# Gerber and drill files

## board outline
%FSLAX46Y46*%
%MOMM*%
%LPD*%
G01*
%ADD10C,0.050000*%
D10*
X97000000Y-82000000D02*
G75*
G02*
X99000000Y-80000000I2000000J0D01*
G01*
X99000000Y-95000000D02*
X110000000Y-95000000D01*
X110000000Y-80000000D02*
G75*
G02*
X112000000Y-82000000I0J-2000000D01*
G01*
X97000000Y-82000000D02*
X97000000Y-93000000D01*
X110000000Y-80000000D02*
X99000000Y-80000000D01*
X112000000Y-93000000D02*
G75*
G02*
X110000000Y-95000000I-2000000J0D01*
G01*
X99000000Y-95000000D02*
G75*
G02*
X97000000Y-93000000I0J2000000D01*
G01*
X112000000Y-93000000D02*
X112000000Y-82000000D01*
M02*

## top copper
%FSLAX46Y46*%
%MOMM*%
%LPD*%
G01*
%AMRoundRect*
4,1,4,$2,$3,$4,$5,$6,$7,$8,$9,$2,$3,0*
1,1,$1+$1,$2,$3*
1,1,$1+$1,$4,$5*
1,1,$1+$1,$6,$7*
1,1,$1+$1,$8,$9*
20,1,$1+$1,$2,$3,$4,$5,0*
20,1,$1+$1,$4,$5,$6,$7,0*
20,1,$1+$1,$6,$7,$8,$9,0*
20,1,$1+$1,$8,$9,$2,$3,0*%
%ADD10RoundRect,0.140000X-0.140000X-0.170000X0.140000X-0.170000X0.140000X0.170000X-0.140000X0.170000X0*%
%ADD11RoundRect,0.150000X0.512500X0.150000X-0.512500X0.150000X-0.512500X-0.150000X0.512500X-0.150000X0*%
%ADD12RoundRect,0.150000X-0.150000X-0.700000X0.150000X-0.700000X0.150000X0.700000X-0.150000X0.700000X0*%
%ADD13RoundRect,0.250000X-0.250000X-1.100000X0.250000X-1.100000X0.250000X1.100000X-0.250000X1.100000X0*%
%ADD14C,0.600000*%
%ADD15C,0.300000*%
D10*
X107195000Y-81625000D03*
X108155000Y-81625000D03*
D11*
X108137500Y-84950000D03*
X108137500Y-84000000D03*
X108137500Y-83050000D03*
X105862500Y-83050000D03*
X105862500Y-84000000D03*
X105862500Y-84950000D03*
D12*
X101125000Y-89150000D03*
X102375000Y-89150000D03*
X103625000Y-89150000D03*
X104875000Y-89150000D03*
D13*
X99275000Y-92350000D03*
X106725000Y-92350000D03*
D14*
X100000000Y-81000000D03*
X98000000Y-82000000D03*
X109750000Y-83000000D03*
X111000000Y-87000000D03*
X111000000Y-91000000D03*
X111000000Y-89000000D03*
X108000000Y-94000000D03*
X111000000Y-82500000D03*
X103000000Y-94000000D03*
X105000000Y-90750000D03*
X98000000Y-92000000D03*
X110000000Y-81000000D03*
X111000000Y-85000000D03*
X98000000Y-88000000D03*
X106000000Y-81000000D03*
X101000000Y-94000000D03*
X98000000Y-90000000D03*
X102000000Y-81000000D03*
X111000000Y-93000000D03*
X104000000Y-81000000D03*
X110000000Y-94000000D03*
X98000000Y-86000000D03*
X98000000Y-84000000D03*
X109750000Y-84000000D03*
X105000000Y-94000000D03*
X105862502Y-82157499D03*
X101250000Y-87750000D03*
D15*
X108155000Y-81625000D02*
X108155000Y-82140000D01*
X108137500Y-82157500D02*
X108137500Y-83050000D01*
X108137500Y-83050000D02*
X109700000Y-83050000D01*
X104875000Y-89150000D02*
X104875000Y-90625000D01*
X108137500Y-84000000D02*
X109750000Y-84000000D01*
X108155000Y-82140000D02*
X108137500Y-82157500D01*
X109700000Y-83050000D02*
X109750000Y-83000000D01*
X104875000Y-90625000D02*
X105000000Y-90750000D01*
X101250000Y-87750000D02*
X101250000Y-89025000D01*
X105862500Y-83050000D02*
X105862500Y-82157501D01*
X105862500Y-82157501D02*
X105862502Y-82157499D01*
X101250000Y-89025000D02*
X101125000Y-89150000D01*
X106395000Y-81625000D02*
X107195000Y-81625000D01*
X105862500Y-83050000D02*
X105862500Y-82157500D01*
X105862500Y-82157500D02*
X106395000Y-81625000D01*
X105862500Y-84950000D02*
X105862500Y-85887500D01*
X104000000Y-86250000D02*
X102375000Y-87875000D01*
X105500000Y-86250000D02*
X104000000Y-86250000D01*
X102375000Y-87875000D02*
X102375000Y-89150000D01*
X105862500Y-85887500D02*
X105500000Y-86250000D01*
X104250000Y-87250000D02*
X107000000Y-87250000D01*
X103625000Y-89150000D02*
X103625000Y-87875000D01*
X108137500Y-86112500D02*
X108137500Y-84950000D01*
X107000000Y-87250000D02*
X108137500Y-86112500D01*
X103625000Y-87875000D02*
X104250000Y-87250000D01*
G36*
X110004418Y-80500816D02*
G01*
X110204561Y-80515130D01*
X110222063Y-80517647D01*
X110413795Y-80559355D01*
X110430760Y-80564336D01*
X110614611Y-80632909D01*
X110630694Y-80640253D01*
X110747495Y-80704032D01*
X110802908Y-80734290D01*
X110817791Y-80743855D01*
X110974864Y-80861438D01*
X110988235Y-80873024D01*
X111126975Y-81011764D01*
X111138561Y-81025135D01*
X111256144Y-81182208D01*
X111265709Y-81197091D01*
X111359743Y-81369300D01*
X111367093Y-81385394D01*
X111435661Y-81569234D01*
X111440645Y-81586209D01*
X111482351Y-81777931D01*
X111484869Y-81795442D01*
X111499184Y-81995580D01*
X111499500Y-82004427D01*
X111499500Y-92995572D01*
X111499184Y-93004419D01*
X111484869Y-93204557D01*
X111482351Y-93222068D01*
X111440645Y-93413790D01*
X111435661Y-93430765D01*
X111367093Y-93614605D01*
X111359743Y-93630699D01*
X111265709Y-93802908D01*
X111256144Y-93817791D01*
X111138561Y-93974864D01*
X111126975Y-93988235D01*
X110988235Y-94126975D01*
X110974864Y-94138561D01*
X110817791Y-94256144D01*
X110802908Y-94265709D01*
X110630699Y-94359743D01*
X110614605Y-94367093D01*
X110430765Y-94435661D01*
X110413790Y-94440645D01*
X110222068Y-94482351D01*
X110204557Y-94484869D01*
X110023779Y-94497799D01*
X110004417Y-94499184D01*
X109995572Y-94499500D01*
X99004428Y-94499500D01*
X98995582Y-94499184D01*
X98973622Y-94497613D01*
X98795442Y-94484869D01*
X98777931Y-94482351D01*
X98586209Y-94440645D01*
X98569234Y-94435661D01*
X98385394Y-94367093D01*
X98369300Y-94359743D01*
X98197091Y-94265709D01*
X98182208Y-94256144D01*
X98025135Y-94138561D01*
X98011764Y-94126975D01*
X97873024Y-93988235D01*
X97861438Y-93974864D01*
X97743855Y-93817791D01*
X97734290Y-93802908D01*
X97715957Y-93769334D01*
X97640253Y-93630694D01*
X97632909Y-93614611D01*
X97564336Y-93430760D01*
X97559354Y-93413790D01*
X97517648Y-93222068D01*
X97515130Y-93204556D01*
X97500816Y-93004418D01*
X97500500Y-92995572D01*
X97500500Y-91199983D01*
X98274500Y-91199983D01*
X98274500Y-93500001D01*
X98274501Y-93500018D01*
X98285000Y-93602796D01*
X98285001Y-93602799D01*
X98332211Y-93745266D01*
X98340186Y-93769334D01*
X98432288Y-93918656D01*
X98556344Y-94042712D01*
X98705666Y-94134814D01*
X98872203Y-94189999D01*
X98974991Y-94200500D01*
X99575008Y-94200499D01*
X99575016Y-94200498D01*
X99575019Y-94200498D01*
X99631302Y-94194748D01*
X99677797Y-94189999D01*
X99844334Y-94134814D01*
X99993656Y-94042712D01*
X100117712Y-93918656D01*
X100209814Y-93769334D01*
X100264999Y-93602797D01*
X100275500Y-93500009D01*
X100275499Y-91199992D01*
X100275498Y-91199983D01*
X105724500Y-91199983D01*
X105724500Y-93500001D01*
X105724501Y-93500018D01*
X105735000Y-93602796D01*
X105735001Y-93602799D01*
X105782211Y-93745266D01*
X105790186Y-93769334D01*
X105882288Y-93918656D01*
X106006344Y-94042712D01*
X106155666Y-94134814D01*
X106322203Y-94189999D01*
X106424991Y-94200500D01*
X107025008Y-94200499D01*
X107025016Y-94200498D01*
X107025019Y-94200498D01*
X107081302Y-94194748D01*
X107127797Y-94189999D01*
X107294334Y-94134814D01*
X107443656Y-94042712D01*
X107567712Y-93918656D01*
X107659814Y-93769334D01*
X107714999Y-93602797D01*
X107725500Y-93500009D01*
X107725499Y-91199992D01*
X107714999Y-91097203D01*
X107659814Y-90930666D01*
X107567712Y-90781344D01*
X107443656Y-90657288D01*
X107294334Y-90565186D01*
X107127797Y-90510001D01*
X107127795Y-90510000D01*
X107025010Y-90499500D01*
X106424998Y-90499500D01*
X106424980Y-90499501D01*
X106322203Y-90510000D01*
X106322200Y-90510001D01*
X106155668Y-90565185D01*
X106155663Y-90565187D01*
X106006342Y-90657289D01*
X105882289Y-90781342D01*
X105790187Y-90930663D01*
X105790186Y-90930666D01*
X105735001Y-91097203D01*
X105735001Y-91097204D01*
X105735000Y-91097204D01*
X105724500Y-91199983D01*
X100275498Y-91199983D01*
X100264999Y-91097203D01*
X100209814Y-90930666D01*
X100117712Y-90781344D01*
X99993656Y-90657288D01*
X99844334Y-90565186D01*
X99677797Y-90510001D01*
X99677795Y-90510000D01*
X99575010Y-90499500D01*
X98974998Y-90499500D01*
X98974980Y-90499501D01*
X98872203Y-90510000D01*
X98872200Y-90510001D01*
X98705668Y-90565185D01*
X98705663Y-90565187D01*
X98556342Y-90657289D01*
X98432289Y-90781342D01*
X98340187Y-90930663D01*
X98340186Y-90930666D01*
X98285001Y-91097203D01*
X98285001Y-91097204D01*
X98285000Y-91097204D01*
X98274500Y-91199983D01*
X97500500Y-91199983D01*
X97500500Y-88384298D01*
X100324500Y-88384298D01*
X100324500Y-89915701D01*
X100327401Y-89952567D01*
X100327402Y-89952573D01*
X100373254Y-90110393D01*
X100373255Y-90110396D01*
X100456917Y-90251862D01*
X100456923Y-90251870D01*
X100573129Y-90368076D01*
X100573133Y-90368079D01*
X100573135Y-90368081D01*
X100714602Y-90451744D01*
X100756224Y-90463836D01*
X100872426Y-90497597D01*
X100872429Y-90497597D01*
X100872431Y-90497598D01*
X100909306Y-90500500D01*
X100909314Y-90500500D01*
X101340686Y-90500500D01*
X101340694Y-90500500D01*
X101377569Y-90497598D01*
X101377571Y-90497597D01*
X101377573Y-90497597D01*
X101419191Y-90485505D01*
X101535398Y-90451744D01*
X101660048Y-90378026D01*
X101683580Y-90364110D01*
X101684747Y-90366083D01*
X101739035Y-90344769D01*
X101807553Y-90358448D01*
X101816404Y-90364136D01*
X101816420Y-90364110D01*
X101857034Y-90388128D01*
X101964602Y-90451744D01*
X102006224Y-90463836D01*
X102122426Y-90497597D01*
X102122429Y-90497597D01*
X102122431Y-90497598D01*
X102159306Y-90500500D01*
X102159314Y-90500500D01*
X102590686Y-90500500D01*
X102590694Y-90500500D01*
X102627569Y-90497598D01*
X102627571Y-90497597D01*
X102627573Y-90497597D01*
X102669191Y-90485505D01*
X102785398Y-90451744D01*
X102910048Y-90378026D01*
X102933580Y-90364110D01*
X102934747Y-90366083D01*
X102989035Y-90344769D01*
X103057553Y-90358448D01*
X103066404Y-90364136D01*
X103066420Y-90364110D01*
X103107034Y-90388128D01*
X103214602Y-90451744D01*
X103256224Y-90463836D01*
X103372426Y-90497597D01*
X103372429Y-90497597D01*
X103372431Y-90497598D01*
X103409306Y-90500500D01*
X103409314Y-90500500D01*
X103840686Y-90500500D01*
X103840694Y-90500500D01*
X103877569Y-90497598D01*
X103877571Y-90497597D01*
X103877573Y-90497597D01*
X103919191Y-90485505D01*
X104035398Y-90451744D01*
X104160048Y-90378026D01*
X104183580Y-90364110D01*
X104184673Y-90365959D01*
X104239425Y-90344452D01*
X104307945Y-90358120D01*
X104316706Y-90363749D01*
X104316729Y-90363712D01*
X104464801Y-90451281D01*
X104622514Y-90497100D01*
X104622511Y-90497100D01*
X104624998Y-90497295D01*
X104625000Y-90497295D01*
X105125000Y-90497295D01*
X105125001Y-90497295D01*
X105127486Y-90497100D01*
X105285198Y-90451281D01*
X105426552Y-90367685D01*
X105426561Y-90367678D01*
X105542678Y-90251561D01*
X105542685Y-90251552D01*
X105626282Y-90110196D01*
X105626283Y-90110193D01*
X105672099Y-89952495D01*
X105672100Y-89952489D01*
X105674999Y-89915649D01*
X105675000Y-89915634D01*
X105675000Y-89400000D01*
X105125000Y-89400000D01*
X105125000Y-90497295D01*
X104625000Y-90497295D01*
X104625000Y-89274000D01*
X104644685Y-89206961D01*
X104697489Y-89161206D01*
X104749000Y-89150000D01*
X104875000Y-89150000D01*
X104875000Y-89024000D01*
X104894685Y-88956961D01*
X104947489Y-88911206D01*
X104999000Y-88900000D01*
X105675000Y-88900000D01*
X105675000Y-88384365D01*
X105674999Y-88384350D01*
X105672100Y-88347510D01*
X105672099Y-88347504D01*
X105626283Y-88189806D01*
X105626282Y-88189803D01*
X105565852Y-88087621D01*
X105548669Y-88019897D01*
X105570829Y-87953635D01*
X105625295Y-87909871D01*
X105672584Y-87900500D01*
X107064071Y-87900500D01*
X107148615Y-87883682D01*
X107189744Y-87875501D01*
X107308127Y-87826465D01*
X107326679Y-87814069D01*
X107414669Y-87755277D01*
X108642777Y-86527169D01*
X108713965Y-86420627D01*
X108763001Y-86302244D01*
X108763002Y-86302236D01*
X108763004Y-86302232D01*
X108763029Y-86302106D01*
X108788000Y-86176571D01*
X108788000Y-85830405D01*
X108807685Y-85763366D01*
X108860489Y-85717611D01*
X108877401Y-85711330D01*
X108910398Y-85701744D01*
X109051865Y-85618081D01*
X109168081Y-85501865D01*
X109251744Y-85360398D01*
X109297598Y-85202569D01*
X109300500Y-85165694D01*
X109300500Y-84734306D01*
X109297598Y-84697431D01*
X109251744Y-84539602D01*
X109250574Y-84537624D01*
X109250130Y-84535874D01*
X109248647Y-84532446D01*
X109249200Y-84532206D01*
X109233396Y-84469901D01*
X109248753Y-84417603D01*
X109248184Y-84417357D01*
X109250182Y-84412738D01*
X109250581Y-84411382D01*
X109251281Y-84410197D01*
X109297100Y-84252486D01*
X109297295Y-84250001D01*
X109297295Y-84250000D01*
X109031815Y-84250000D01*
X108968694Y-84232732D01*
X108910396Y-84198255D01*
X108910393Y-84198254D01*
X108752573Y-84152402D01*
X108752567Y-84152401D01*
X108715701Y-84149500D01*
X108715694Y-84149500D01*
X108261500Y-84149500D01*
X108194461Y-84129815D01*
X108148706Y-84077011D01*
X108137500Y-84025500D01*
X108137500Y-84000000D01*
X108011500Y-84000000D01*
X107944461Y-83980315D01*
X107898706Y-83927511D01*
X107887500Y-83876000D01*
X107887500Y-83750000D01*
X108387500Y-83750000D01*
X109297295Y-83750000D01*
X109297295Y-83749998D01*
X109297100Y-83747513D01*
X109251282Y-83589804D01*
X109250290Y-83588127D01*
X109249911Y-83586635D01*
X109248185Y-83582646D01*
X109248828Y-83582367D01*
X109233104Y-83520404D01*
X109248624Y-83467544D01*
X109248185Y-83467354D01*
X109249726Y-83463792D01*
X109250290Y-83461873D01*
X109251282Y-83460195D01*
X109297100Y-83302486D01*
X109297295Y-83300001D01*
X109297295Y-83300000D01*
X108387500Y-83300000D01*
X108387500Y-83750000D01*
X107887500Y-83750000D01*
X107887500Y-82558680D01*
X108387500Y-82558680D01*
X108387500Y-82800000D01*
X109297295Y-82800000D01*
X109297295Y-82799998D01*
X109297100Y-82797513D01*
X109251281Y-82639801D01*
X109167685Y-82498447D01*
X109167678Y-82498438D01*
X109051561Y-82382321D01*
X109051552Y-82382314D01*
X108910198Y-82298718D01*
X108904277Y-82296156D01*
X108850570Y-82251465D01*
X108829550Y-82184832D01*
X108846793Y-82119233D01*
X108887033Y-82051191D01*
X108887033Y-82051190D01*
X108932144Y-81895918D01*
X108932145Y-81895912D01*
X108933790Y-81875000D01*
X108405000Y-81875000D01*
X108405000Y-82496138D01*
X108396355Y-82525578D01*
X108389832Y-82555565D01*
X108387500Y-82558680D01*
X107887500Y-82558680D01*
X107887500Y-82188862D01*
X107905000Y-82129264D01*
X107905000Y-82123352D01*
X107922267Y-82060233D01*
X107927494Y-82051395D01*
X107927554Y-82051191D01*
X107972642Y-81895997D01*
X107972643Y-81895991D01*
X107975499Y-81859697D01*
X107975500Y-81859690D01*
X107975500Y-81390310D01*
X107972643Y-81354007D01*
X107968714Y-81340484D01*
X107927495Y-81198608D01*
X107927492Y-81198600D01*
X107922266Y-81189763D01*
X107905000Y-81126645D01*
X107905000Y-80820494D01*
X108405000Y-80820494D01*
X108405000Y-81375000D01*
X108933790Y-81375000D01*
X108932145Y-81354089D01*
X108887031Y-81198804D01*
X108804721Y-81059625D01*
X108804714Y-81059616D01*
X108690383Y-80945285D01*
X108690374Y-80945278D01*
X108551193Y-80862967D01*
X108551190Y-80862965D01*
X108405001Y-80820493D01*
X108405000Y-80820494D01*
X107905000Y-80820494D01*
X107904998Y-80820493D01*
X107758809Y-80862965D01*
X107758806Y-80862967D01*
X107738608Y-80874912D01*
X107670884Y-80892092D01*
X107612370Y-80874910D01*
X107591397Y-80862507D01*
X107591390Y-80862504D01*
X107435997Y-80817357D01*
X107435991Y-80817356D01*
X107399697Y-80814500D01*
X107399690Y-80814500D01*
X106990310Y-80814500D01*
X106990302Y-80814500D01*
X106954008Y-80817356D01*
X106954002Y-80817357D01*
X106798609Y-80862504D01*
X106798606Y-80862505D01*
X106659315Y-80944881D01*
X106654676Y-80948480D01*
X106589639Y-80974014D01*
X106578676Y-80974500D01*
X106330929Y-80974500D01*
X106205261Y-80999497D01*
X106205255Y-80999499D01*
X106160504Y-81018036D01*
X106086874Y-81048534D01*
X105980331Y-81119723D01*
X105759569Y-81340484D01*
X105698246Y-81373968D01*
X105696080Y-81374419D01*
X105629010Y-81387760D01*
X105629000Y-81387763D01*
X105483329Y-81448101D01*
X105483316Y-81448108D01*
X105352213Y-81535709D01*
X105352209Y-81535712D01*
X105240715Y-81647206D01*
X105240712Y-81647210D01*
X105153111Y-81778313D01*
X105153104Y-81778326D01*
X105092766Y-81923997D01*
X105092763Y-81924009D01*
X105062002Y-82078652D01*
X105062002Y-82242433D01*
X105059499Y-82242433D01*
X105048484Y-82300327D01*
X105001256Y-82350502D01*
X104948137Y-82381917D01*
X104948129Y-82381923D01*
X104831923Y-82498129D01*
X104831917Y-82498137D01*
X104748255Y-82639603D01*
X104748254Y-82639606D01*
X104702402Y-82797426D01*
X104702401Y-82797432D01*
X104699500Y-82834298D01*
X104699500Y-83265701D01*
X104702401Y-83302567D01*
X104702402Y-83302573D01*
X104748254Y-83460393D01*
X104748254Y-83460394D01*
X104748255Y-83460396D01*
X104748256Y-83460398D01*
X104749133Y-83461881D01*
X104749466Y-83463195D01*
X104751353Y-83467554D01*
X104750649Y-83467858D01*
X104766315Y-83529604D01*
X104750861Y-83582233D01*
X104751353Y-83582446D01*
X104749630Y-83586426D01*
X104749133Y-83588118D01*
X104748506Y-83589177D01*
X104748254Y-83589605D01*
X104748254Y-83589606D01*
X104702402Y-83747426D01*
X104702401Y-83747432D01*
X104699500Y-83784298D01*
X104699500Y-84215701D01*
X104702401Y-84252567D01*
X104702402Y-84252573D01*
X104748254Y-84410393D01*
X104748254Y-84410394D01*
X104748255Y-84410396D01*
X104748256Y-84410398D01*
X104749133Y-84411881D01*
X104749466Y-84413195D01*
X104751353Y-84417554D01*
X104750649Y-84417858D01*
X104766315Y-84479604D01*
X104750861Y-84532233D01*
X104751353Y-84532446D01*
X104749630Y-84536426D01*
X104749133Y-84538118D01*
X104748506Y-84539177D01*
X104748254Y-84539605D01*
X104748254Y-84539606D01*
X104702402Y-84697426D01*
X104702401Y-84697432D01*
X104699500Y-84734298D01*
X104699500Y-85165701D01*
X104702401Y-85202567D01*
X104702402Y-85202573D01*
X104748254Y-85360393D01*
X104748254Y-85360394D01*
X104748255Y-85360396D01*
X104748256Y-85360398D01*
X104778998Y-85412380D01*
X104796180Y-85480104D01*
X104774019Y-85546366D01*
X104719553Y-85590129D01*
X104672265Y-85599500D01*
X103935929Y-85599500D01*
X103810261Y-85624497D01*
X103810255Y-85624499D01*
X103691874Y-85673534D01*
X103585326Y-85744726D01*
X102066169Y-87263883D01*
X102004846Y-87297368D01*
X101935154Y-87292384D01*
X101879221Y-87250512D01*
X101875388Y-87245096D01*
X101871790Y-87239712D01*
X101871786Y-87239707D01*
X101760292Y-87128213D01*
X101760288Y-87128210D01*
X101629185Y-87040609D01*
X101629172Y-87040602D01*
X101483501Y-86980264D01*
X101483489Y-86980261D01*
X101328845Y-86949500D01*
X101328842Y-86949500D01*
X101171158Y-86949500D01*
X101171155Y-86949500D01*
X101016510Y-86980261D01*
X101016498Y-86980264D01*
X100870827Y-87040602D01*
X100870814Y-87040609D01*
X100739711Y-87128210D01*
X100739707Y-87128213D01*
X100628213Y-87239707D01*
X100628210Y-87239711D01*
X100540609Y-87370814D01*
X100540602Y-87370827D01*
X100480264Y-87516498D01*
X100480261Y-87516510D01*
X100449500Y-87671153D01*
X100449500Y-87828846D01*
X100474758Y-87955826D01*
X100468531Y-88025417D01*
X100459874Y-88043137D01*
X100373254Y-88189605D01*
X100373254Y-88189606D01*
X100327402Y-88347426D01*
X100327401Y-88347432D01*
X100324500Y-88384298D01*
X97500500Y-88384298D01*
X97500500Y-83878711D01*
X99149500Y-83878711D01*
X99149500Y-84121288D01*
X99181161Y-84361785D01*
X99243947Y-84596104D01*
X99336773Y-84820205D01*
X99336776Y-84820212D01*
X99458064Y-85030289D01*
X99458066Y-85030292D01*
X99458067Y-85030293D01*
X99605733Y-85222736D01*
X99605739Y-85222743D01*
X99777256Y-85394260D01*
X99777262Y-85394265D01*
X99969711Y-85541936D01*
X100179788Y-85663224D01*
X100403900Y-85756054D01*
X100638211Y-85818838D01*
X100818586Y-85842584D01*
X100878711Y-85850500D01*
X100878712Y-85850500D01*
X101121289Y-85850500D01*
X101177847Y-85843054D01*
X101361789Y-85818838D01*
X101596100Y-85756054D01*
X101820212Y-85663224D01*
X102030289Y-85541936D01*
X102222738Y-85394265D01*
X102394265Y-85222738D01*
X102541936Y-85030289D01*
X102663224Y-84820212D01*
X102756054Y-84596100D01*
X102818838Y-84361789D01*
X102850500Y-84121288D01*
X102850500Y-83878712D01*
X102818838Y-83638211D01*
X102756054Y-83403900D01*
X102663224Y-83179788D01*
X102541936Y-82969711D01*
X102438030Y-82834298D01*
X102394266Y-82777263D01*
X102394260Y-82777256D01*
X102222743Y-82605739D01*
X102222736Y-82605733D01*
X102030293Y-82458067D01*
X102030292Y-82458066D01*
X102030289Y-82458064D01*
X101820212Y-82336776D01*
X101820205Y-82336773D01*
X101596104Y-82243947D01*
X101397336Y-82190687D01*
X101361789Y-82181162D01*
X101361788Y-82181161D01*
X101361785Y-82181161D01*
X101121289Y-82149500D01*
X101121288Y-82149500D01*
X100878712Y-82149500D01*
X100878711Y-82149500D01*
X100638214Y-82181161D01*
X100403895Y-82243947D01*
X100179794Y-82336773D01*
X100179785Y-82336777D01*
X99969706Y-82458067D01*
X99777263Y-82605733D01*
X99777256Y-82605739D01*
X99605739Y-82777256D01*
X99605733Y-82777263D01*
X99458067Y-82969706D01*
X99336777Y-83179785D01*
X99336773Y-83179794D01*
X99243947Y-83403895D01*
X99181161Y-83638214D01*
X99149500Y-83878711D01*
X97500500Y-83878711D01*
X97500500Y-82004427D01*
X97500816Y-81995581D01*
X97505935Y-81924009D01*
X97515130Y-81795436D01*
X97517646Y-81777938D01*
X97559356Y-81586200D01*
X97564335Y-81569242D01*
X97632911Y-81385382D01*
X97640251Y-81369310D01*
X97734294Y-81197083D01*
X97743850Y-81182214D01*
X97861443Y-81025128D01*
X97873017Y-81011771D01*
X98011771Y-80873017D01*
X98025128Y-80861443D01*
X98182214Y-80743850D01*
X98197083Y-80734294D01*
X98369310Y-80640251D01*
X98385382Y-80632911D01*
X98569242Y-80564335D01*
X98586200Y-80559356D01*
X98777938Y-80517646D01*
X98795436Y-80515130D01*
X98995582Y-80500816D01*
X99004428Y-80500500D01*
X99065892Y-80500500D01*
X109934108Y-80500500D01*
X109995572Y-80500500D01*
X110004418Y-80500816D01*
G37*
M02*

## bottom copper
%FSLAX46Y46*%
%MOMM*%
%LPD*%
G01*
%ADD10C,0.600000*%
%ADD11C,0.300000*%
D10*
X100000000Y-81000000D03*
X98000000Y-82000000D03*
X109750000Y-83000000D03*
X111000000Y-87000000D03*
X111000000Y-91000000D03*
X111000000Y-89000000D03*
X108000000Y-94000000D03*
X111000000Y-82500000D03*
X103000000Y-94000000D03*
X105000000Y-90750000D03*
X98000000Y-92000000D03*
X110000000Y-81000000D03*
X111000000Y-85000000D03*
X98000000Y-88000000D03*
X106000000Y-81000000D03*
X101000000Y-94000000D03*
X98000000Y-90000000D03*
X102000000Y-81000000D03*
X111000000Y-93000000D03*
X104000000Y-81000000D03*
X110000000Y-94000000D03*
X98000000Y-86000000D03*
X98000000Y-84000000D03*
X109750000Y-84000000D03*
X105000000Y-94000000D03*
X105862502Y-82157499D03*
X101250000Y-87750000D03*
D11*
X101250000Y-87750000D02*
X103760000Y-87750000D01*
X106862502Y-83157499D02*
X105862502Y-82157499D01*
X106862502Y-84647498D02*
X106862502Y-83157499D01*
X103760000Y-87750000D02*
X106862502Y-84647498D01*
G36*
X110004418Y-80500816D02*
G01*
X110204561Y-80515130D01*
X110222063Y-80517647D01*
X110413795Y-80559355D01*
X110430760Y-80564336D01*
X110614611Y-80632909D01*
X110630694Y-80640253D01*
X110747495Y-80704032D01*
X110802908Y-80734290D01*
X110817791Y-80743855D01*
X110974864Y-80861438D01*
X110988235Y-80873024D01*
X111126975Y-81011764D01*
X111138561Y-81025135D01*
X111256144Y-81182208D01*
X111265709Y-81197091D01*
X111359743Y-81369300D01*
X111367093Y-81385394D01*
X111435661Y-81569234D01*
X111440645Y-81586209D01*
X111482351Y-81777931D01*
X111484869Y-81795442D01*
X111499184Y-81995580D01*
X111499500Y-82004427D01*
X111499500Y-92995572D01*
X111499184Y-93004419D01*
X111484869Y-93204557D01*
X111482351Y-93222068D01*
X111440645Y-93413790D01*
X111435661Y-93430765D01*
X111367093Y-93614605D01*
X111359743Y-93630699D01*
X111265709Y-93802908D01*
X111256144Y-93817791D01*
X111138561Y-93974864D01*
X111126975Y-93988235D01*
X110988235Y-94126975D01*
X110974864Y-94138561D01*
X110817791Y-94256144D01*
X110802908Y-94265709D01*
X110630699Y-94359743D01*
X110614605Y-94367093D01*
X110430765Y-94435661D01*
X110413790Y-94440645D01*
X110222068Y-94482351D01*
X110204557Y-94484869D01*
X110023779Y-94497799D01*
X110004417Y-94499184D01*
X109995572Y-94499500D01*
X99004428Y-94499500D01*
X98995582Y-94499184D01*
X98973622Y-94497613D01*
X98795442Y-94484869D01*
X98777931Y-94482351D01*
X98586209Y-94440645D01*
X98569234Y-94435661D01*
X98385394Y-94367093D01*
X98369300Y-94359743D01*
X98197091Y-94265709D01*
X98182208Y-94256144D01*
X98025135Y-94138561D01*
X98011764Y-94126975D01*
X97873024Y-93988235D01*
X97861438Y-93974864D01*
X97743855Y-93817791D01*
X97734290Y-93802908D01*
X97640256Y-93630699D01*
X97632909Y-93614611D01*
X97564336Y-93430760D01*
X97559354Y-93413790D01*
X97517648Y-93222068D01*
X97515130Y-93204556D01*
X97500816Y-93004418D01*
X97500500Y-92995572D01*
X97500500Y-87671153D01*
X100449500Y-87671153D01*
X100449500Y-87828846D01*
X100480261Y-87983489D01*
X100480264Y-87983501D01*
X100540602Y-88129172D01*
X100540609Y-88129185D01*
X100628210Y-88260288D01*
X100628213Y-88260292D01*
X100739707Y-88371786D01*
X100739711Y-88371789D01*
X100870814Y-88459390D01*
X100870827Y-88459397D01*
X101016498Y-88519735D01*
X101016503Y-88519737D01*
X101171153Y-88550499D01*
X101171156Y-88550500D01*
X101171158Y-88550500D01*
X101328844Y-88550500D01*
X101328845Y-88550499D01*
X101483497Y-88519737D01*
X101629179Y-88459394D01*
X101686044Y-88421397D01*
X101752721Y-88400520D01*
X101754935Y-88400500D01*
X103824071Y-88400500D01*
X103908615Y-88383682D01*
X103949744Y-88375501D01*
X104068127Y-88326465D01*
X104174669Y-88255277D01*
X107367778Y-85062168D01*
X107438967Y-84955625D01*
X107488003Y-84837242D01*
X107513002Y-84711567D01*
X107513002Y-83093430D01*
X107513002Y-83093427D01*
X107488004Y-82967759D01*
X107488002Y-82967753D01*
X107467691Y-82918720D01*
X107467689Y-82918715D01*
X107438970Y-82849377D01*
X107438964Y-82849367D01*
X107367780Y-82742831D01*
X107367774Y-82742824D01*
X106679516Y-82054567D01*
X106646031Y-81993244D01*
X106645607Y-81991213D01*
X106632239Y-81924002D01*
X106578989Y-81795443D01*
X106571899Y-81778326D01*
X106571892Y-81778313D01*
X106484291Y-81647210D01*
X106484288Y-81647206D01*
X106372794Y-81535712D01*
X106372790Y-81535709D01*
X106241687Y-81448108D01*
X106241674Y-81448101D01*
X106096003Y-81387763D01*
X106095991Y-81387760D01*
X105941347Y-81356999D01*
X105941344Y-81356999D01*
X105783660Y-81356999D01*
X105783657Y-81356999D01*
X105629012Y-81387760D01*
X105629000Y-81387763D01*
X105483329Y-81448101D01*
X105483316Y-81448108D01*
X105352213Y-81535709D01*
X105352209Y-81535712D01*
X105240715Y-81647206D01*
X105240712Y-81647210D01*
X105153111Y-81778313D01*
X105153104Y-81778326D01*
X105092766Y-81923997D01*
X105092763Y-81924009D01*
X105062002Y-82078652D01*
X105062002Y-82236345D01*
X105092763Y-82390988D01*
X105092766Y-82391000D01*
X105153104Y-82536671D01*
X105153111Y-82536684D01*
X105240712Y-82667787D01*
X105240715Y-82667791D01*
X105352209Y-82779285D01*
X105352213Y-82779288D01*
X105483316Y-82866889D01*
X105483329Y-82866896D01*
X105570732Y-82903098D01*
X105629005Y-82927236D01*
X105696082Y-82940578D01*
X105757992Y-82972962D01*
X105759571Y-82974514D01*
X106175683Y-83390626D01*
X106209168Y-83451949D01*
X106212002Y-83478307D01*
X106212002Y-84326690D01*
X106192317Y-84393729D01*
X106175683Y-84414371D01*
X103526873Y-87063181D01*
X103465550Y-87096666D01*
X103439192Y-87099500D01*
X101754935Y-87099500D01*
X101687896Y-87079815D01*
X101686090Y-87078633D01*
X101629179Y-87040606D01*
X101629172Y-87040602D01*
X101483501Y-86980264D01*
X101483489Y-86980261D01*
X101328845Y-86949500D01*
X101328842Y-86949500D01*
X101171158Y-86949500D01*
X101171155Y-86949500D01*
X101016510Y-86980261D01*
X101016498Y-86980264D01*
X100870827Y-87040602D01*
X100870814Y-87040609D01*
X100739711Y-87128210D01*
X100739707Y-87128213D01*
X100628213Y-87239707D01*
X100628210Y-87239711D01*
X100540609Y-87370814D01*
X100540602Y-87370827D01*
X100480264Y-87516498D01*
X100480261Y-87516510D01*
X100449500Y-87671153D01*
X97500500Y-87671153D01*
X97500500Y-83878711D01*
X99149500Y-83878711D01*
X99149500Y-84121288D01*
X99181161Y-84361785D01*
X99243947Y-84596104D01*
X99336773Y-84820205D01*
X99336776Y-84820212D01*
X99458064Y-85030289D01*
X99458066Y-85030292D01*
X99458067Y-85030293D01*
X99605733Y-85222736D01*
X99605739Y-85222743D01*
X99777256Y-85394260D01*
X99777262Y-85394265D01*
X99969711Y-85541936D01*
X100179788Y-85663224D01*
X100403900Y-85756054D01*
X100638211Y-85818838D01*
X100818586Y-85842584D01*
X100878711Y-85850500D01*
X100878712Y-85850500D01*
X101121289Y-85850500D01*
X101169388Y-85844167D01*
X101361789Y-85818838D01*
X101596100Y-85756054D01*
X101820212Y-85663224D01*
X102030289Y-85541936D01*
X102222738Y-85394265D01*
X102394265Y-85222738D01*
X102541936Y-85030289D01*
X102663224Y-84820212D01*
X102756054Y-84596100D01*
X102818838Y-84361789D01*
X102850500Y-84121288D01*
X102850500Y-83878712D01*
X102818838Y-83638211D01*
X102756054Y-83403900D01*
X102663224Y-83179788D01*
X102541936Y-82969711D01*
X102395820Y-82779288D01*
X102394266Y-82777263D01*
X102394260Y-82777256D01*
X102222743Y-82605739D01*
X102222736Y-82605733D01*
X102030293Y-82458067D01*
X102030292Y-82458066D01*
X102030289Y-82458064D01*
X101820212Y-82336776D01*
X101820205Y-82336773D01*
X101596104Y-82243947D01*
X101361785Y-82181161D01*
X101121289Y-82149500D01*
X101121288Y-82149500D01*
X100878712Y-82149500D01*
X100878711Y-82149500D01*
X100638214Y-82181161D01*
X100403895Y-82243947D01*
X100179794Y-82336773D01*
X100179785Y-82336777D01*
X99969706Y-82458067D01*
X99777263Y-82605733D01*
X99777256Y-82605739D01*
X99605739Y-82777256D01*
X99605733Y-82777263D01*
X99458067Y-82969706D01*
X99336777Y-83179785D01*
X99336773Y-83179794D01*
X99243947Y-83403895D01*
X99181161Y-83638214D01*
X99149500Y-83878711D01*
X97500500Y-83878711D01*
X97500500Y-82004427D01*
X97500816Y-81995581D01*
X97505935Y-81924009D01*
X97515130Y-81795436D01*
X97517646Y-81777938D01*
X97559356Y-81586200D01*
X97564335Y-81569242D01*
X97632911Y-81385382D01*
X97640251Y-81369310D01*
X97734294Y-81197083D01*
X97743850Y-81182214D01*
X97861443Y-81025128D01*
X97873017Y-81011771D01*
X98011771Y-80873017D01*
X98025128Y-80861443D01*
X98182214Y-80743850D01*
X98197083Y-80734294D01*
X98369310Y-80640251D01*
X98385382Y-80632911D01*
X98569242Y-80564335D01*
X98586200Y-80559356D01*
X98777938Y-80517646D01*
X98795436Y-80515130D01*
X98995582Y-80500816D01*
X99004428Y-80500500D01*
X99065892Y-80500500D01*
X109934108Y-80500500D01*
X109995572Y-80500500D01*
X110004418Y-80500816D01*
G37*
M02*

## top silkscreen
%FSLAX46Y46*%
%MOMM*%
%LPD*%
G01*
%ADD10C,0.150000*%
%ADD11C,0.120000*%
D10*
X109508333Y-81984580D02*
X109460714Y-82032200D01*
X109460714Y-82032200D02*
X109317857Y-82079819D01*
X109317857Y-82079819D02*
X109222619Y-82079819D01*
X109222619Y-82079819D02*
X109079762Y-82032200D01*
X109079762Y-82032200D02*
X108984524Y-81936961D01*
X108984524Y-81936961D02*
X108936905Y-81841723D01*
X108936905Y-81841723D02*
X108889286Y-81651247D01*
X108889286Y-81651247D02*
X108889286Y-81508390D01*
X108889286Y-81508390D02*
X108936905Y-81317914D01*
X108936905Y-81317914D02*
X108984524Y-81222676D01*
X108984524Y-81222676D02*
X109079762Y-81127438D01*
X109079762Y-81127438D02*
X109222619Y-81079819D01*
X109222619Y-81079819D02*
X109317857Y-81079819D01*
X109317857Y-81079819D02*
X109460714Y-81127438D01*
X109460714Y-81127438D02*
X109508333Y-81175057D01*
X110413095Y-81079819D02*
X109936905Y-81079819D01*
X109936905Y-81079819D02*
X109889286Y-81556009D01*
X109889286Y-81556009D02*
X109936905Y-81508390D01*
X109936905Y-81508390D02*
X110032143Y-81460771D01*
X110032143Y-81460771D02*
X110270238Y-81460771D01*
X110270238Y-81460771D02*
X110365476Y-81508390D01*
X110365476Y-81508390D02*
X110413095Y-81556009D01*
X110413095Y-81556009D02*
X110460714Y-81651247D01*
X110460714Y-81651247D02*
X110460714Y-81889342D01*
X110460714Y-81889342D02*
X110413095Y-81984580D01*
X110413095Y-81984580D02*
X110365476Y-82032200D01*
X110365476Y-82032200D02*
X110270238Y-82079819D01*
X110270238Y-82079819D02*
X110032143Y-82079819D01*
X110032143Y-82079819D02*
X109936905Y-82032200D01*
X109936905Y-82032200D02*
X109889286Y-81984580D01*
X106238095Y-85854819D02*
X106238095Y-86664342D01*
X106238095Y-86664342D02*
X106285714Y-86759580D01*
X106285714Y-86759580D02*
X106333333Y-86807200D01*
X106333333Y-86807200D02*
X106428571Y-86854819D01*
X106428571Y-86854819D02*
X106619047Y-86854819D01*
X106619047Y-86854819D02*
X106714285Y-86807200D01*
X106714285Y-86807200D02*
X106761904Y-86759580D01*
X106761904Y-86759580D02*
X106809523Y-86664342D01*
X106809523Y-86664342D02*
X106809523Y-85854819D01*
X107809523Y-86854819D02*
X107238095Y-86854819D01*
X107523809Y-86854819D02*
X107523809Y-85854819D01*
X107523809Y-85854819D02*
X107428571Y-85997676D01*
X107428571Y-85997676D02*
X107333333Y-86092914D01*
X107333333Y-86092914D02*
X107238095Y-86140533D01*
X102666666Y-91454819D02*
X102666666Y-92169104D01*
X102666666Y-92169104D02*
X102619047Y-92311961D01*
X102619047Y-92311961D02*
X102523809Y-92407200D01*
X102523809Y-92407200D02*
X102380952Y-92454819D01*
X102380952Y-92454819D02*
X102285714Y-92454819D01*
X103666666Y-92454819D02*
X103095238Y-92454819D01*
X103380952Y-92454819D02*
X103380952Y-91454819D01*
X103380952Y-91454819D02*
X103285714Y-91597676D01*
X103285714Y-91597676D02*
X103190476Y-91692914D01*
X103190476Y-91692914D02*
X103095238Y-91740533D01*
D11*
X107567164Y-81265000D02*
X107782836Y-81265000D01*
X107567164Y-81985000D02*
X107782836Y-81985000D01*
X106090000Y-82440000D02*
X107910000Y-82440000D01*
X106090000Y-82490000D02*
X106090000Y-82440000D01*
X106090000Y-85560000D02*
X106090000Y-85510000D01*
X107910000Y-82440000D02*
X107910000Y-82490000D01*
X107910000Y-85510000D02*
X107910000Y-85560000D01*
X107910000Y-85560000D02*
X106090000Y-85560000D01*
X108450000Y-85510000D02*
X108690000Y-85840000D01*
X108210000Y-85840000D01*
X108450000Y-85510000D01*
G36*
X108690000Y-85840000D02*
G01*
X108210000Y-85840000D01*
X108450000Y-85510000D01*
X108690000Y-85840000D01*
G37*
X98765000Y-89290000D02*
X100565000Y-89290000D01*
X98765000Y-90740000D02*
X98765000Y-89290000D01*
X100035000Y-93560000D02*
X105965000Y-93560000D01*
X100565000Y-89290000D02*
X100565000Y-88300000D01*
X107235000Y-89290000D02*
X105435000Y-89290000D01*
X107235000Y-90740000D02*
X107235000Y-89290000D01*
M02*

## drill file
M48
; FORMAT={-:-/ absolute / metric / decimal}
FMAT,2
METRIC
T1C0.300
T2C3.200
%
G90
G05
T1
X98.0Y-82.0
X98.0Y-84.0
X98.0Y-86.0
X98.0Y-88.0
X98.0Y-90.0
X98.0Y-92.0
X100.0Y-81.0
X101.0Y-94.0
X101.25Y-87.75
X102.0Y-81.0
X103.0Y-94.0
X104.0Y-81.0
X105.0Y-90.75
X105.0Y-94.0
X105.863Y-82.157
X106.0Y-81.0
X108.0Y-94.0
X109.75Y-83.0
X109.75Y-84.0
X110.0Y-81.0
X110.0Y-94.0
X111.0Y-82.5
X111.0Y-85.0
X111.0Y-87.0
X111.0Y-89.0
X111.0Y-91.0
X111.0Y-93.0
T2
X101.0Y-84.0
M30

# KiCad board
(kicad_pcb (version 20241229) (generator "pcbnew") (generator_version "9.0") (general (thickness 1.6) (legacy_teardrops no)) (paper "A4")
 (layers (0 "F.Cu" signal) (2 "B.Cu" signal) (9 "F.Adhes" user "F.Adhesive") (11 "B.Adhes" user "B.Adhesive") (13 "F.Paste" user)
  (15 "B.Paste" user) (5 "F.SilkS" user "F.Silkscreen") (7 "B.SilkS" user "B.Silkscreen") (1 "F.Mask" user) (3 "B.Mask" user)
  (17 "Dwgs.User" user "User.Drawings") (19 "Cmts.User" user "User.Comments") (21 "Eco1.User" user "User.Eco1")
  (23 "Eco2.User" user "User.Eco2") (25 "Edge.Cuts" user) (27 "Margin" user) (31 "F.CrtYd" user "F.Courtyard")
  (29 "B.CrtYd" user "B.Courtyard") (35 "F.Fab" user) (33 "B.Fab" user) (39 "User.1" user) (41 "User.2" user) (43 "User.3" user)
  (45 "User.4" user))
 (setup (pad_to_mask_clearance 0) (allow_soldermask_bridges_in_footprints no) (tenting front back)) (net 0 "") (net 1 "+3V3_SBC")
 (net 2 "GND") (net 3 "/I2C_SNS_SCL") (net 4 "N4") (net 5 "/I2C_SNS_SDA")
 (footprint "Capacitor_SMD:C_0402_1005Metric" (layer "F.Cu") (at 107.675 81.625)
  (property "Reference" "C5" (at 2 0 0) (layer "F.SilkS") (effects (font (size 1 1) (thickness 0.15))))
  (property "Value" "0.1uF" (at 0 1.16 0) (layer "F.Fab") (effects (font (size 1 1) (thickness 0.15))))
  (fp_line (start -0.107836 -0.36) (end 0.107836 -0.36) (stroke (width 0.12) (type solid)) (layer "F.SilkS"))
  (fp_line (start -0.107836 0.36) (end 0.107836 0.36) (stroke (width 0.12) (type solid)) (layer "F.SilkS"))
  (pad "1" smd roundrect (at -0.48 0) (size 0.56 0.62) (layers "F.Cu" "F.Mask" "F.Paste") (roundrect_rratio 0.25) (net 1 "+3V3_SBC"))
  (pad "2" smd roundrect (at 0.48 0) (size 0.56 0.62) (layers "F.Cu" "F.Mask" "F.Paste") (roundrect_rratio 0.25) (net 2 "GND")))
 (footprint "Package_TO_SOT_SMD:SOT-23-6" (layer "F.Cu") (at 107 84 180)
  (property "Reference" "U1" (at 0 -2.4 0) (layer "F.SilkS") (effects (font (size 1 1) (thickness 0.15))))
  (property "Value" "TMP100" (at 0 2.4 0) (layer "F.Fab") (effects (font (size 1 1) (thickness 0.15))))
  (fp_line (start 0.91 1.56) (end -0.91 1.56) (stroke (width 0.12) (type solid)) (layer "F.SilkS"))
  (fp_line (start 0.91 1.51) (end 0.91 1.56) (stroke (width 0.12) (type solid)) (layer "F.SilkS"))
  (fp_line (start 0.91 -1.56) (end 0.91 -1.51) (stroke (width 0.12) (type solid)) (layer "F.SilkS"))
  (fp_line (start -0.91 1.56) (end -0.91 1.51) (stroke (width 0.12) (type solid)) (layer "F.SilkS"))
  (fp_line (start -0.91 -1.51) (end -0.91 -1.56) (stroke (width 0.12) (type solid)) (layer "F.SilkS"))
  (fp_line (start -0.91 -1.56) (end 0.91 -1.56) (stroke (width 0.12) (type solid)) (layer "F.SilkS"))
  (fp_poly (pts (xy -1.45 -1.51) (xy -1.69 -1.84) (xy -1.21 -1.84)) (stroke (width 0.12) (type solid)) (fill yes) (layer "F.SilkS"))
  (pad "1" smd roundrect (at -1.1375 -0.95 180) (size 1.325 0.6) (layers "F.Cu" "F.Mask" "F.Paste") (roundrect_rratio 0.25)
   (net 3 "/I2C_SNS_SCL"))
  (pad "2" smd roundrect (at -1.1375 0 180) (size 1.325 0.6) (layers "F.Cu" "F.Mask" "F.Paste") (roundrect_rratio 0.25) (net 2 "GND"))
  (pad "3" smd roundrect (at -1.1375 0.95 180) (size 1.325 0.6) (layers "F.Cu" "F.Mask" "F.Paste") (roundrect_rratio 0.25) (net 2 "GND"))
  (pad "4" smd roundrect (at 1.1375 0.95 180) (size 1.325 0.6) (layers "F.Cu" "F.Mask" "F.Paste") (roundrect_rratio 0.25) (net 1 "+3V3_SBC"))
  (pad "5" smd roundrect (at 1.1375 0 180) (size 1.325 0.6) (layers "F.Cu" "F.Mask" "F.Paste") (roundrect_rratio 0.25) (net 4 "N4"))
  (pad "6" smd roundrect (at 1.1375 -0.95 180) (size 1.325 0.6) (layers "F.Cu" "F.Mask" "F.Paste") (roundrect_rratio 0.25)
   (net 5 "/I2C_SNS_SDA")))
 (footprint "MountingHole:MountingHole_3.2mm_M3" (layer "F.Cu") (at 101 84)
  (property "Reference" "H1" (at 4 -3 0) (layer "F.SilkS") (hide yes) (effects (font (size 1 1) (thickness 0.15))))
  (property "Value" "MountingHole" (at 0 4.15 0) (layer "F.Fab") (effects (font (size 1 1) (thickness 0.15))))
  (pad "" np_thru_hole circle (at 0 0) (size 3.2 3.2) (drill 3.2) (layers "*.Cu" "*.Mask")))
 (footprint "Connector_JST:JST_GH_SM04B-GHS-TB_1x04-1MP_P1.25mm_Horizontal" (layer "F.Cu") (at 103 91)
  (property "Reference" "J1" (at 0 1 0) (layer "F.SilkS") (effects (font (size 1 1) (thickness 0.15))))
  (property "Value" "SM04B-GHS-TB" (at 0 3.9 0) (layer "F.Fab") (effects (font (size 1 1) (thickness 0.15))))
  (fp_line (start -4.235 -1.71) (end -2.435 -1.71) (stroke (width 0.12) (type solid)) (layer "F.SilkS"))
  (fp_line (start -4.235 -0.26) (end -4.235 -1.71) (stroke (width 0.12) (type solid)) (layer "F.SilkS"))
  (fp_line (start -2.965 2.56) (end 2.965 2.56) (stroke (width 0.12) (type solid)) (layer "F.SilkS"))
  (fp_line (start -2.435 -1.71) (end -2.435 -2.7) (stroke (width 0.12) (type solid)) (layer "F.SilkS"))
  (fp_line (start 4.235 -1.71) (end 2.435 -1.71) (stroke (width 0.12) (type solid)) (layer "F.SilkS"))
  (fp_line (start 4.235 -0.26) (end 4.235 -1.71) (stroke (width 0.12) (type solid)) (layer "F.SilkS"))
  (pad "1" smd roundrect (at -1.875 -1.85) (size 0.6 1.7) (layers "F.Cu" "F.Mask" "F.Paste") (roundrect_rratio 0.25) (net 1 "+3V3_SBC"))
  (pad "2" smd roundrect (at -0.625 -1.85) (size 0.6 1.7) (layers "F.Cu" "F.Mask" "F.Paste") (roundrect_rratio 0.25) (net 5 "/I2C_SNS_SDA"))
  (pad "3" smd roundrect (at 0.625 -1.85) (size 0.6 1.7) (layers "F.Cu" "F.Mask" "F.Paste") (roundrect_rratio 0.25) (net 3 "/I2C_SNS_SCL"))
  (pad "4" smd roundrect (at 1.875 -1.85) (size 0.6 1.7) (layers "F.Cu" "F.Mask" "F.Paste") (roundrect_rratio 0.25) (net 2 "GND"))
  (pad "MP" smd roundrect (at -3.725 1.35) (size 1 2.7) (layers "F.Cu" "F.Mask" "F.Paste") (roundrect_rratio 0.25))
  (pad "MP" smd roundrect (at 3.725 1.35) (size 1 2.7) (layers "F.Cu" "F.Mask" "F.Paste") (roundrect_rratio 0.25)))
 (gr_arc (start 97 82) (mid 97.585786 80.585786) (end 99 80) (stroke (width 0.05) (type default)) (layer "Edge.Cuts"))
 (gr_line (start 99 95) (end 110 95) (stroke (width 0.05) (type default)) (layer "Edge.Cuts"))
 (gr_arc (start 110 80) (mid 111.414214 80.585786) (end 112 82) (stroke (width 0.05) (type default)) (layer "Edge.Cuts"))
 (gr_line (start 97 82) (end 97 93) (stroke (width 0.05) (type default)) (layer "Edge.Cuts"))
 (gr_line (start 110 80) (end 99 80) (stroke (width 0.05) (type default)) (layer "Edge.Cuts"))
 (gr_arc (start 112 93) (mid 111.414214 94.414214) (end 110 95) (stroke (width 0.05) (type default)) (layer "Edge.Cuts"))
 (gr_arc (start 99 95) (mid 97.585786 94.414214) (end 97 93) (stroke (width 0.05) (type default)) (layer "Edge.Cuts"))
 (gr_line (start 112 93) (end 112 82) (stroke (width 0.05) (type default)) (layer "Edge.Cuts"))
 (segment (start 108.155 81.625) (end 108.155 82.14) (width 0.3) (layer "F.Cu") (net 2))
 (segment (start 108.1375 82.1575) (end 108.1375 83.05) (width 0.3) (layer "F.Cu") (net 2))
 (segment (start 108.1375 83.05) (end 109.7 83.05) (width 0.3) (layer "F.Cu") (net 2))
 (segment (start 104.875 89.15) (end 104.875 90.625) (width 0.3) (layer "F.Cu") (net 2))
 (segment (start 108.1375 84) (end 109.75 84) (width 0.3) (layer "F.Cu") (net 2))
 (segment (start 108.155 82.14) (end 108.1375 82.1575) (width 0.3) (layer "F.Cu") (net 2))
 (segment (start 109.7 83.05) (end 109.75 83) (width 0.3) (layer "F.Cu") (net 2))
 (segment (start 104.875 90.625) (end 105 90.75) (width 0.3) (layer "F.Cu") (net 2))
 (via (at 100 81) (size 0.6) (drill 0.3) (layers "F.Cu" "B.Cu") (free yes) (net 2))
 (via (at 98 82) (size 0.6) (drill 0.3) (layers "F.Cu" "B.Cu") (free yes) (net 2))
 (via (at 109.75 83) (size 0.6) (drill 0.3) (layers "F.Cu" "B.Cu") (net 2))
 (via (at 111 87) (size 0.6) (drill 0.3) (layers "F.Cu" "B.Cu") (free yes) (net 2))
 (via (at 111 91) (size 0.6) (drill 0.3) (layers "F.Cu" "B.Cu") (free yes) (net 2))
 (via (at 111 89) (size 0.6) (drill 0.3) (layers "F.Cu" "B.Cu") (free yes) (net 2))
 (via (at 108 94) (size 0.6) (drill 0.3) (layers "F.Cu" "B.Cu") (free yes) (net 2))
 (via (at 111 82.5) (size 0.6) (drill 0.3) (layers "F.Cu" "B.Cu") (free yes) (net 2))
 (via (at 103 94) (size 0.6) (drill 0.3) (layers "F.Cu" "B.Cu") (free yes) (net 2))
 (via (at 105 90.75) (size 0.6) (drill 0.3) (layers "F.Cu" "B.Cu") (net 2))
 (via (at 98 92) (size 0.6) (drill 0.3) (layers "F.Cu" "B.Cu") (free yes) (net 2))
 (via (at 110 81) (size 0.6) (drill 0.3) (layers "F.Cu" "B.Cu") (free yes) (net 2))
 (via (at 111 85) (size 0.6) (drill 0.3) (layers "F.Cu" "B.Cu") (free yes) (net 2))
 (via (at 98 88) (size 0.6) (drill 0.3) (layers "F.Cu" "B.Cu") (free yes) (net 2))
 (via (at 106 81) (size 0.6) (drill 0.3) (layers "F.Cu" "B.Cu") (free yes) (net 2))
 (via (at 101 94) (size 0.6) (drill 0.3) (layers "F.Cu" "B.Cu") (free yes) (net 2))
 (via (at 98 90) (size 0.6) (drill 0.3) (layers "F.Cu" "B.Cu") (free yes) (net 2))
 (via (at 102 81) (size 0.6) (drill 0.3) (layers "F.Cu" "B.Cu") (free yes) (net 2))
 (via (at 111 93) (size 0.6) (drill 0.3) (layers "F.Cu" "B.Cu") (free yes) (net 2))
 (via (at 104 81) (size 0.6) (drill 0.3) (layers "F.Cu" "B.Cu") (free yes) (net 2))
 (via (at 110 94) (size 0.6) (drill 0.3) (layers "F.Cu" "B.Cu") (free yes) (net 2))
 (via (at 98 86) (size 0.6) (drill 0.3) (layers "F.Cu" "B.Cu") (free yes) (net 2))
 (via (at 98 84) (size 0.6) (drill 0.3) (layers "F.Cu" "B.Cu") (free yes) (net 2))
 (via (at 109.75 84) (size 0.6) (drill 0.3) (layers "F.Cu" "B.Cu") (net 2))
 (via (at 105 94) (size 0.6) (drill 0.3) (layers "F.Cu" "B.Cu") (free yes) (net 2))
 (segment (start 101.25 87.75) (end 101.25 89.025) (width 0.3) (layer "F.Cu") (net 1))
 (segment (start 105.8625 83.05) (end 105.8625 82.157501) (width 0.3) (layer "F.Cu") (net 1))
 (segment (start 105.8625 82.157501) (end 105.862502 82.157499) (width 0.3) (layer "F.Cu") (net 1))
 (segment (start 101.25 89.025) (end 101.125 89.15) (width 0.3) (layer "F.Cu") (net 1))
 (segment (start 106.395 81.625) (end 107.195 81.625) (width 0.3) (layer "F.Cu") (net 1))
 (segment (start 105.8625 83.05) (end 105.8625 82.1575) (width 0.3) (layer "F.Cu") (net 1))
 (segment (start 105.8625 82.1575) (end 106.395 81.625) (width 0.3) (layer "F.Cu") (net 1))
 (via (at 105.862502 82.157499) (size 0.6) (drill 0.3) (layers "F.Cu" "B.Cu") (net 1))
 (via (at 101.25 87.75) (size 0.6) (drill 0.3) (layers "F.Cu" "B.Cu") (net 1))
 (segment (start 101.25 87.75) (end 103.76 87.75) (width 0.3) (layer "B.Cu") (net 1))
 (segment (start 106.862502 83.157499) (end 105.862502 82.157499) (width 0.3) (layer "B.Cu") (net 1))
 (segment (start 106.862502 84.647498) (end 106.862502 83.157499) (width 0.3) (layer "B.Cu") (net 1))
 (segment (start 103.76 87.75) (end 106.862502 84.647498) (width 0.3) (layer "B.Cu") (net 1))
 (segment (start 105.8625 84.95) (end 105.8625 85.8875) (width 0.3) (layer "F.Cu") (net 5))
 (segment (start 104 86.25) (end 102.375 87.875) (width 0.3) (layer "F.Cu") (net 5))
 (segment (start 105.5 86.25) (end 104 86.25) (width 0.3) (layer "F.Cu") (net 5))
 (segment (start 102.375 87.875) (end 102.375 89.15) (width 0.3) (layer "F.Cu") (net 5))
 (segment (start 105.8625 85.8875) (end 105.5 86.25) (width 0.3) (layer "F.Cu") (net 5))
 (segment (start 104.25 87.25) (end 107 87.25) (width 0.3) (layer "F.Cu") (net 3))
 (segment (start 103.625 89.15) (end 103.625 87.875) (width 0.3) (layer "F.Cu") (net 3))
 (segment (start 108.1375 86.1125) (end 108.1375 84.95) (width 0.3) (layer "F.Cu") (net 3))
 (segment (start 107 87.25) (end 108.1375 86.1125) (width 0.3) (layer "F.Cu") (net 3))
 (segment (start 103.625 87.875) (end 104.25 87.25) (width 0.3) (layer "F.Cu") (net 3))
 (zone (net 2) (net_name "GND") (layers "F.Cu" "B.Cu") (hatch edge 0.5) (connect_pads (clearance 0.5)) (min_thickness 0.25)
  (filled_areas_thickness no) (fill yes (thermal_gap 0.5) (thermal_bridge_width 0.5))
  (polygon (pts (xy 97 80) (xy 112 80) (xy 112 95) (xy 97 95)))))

